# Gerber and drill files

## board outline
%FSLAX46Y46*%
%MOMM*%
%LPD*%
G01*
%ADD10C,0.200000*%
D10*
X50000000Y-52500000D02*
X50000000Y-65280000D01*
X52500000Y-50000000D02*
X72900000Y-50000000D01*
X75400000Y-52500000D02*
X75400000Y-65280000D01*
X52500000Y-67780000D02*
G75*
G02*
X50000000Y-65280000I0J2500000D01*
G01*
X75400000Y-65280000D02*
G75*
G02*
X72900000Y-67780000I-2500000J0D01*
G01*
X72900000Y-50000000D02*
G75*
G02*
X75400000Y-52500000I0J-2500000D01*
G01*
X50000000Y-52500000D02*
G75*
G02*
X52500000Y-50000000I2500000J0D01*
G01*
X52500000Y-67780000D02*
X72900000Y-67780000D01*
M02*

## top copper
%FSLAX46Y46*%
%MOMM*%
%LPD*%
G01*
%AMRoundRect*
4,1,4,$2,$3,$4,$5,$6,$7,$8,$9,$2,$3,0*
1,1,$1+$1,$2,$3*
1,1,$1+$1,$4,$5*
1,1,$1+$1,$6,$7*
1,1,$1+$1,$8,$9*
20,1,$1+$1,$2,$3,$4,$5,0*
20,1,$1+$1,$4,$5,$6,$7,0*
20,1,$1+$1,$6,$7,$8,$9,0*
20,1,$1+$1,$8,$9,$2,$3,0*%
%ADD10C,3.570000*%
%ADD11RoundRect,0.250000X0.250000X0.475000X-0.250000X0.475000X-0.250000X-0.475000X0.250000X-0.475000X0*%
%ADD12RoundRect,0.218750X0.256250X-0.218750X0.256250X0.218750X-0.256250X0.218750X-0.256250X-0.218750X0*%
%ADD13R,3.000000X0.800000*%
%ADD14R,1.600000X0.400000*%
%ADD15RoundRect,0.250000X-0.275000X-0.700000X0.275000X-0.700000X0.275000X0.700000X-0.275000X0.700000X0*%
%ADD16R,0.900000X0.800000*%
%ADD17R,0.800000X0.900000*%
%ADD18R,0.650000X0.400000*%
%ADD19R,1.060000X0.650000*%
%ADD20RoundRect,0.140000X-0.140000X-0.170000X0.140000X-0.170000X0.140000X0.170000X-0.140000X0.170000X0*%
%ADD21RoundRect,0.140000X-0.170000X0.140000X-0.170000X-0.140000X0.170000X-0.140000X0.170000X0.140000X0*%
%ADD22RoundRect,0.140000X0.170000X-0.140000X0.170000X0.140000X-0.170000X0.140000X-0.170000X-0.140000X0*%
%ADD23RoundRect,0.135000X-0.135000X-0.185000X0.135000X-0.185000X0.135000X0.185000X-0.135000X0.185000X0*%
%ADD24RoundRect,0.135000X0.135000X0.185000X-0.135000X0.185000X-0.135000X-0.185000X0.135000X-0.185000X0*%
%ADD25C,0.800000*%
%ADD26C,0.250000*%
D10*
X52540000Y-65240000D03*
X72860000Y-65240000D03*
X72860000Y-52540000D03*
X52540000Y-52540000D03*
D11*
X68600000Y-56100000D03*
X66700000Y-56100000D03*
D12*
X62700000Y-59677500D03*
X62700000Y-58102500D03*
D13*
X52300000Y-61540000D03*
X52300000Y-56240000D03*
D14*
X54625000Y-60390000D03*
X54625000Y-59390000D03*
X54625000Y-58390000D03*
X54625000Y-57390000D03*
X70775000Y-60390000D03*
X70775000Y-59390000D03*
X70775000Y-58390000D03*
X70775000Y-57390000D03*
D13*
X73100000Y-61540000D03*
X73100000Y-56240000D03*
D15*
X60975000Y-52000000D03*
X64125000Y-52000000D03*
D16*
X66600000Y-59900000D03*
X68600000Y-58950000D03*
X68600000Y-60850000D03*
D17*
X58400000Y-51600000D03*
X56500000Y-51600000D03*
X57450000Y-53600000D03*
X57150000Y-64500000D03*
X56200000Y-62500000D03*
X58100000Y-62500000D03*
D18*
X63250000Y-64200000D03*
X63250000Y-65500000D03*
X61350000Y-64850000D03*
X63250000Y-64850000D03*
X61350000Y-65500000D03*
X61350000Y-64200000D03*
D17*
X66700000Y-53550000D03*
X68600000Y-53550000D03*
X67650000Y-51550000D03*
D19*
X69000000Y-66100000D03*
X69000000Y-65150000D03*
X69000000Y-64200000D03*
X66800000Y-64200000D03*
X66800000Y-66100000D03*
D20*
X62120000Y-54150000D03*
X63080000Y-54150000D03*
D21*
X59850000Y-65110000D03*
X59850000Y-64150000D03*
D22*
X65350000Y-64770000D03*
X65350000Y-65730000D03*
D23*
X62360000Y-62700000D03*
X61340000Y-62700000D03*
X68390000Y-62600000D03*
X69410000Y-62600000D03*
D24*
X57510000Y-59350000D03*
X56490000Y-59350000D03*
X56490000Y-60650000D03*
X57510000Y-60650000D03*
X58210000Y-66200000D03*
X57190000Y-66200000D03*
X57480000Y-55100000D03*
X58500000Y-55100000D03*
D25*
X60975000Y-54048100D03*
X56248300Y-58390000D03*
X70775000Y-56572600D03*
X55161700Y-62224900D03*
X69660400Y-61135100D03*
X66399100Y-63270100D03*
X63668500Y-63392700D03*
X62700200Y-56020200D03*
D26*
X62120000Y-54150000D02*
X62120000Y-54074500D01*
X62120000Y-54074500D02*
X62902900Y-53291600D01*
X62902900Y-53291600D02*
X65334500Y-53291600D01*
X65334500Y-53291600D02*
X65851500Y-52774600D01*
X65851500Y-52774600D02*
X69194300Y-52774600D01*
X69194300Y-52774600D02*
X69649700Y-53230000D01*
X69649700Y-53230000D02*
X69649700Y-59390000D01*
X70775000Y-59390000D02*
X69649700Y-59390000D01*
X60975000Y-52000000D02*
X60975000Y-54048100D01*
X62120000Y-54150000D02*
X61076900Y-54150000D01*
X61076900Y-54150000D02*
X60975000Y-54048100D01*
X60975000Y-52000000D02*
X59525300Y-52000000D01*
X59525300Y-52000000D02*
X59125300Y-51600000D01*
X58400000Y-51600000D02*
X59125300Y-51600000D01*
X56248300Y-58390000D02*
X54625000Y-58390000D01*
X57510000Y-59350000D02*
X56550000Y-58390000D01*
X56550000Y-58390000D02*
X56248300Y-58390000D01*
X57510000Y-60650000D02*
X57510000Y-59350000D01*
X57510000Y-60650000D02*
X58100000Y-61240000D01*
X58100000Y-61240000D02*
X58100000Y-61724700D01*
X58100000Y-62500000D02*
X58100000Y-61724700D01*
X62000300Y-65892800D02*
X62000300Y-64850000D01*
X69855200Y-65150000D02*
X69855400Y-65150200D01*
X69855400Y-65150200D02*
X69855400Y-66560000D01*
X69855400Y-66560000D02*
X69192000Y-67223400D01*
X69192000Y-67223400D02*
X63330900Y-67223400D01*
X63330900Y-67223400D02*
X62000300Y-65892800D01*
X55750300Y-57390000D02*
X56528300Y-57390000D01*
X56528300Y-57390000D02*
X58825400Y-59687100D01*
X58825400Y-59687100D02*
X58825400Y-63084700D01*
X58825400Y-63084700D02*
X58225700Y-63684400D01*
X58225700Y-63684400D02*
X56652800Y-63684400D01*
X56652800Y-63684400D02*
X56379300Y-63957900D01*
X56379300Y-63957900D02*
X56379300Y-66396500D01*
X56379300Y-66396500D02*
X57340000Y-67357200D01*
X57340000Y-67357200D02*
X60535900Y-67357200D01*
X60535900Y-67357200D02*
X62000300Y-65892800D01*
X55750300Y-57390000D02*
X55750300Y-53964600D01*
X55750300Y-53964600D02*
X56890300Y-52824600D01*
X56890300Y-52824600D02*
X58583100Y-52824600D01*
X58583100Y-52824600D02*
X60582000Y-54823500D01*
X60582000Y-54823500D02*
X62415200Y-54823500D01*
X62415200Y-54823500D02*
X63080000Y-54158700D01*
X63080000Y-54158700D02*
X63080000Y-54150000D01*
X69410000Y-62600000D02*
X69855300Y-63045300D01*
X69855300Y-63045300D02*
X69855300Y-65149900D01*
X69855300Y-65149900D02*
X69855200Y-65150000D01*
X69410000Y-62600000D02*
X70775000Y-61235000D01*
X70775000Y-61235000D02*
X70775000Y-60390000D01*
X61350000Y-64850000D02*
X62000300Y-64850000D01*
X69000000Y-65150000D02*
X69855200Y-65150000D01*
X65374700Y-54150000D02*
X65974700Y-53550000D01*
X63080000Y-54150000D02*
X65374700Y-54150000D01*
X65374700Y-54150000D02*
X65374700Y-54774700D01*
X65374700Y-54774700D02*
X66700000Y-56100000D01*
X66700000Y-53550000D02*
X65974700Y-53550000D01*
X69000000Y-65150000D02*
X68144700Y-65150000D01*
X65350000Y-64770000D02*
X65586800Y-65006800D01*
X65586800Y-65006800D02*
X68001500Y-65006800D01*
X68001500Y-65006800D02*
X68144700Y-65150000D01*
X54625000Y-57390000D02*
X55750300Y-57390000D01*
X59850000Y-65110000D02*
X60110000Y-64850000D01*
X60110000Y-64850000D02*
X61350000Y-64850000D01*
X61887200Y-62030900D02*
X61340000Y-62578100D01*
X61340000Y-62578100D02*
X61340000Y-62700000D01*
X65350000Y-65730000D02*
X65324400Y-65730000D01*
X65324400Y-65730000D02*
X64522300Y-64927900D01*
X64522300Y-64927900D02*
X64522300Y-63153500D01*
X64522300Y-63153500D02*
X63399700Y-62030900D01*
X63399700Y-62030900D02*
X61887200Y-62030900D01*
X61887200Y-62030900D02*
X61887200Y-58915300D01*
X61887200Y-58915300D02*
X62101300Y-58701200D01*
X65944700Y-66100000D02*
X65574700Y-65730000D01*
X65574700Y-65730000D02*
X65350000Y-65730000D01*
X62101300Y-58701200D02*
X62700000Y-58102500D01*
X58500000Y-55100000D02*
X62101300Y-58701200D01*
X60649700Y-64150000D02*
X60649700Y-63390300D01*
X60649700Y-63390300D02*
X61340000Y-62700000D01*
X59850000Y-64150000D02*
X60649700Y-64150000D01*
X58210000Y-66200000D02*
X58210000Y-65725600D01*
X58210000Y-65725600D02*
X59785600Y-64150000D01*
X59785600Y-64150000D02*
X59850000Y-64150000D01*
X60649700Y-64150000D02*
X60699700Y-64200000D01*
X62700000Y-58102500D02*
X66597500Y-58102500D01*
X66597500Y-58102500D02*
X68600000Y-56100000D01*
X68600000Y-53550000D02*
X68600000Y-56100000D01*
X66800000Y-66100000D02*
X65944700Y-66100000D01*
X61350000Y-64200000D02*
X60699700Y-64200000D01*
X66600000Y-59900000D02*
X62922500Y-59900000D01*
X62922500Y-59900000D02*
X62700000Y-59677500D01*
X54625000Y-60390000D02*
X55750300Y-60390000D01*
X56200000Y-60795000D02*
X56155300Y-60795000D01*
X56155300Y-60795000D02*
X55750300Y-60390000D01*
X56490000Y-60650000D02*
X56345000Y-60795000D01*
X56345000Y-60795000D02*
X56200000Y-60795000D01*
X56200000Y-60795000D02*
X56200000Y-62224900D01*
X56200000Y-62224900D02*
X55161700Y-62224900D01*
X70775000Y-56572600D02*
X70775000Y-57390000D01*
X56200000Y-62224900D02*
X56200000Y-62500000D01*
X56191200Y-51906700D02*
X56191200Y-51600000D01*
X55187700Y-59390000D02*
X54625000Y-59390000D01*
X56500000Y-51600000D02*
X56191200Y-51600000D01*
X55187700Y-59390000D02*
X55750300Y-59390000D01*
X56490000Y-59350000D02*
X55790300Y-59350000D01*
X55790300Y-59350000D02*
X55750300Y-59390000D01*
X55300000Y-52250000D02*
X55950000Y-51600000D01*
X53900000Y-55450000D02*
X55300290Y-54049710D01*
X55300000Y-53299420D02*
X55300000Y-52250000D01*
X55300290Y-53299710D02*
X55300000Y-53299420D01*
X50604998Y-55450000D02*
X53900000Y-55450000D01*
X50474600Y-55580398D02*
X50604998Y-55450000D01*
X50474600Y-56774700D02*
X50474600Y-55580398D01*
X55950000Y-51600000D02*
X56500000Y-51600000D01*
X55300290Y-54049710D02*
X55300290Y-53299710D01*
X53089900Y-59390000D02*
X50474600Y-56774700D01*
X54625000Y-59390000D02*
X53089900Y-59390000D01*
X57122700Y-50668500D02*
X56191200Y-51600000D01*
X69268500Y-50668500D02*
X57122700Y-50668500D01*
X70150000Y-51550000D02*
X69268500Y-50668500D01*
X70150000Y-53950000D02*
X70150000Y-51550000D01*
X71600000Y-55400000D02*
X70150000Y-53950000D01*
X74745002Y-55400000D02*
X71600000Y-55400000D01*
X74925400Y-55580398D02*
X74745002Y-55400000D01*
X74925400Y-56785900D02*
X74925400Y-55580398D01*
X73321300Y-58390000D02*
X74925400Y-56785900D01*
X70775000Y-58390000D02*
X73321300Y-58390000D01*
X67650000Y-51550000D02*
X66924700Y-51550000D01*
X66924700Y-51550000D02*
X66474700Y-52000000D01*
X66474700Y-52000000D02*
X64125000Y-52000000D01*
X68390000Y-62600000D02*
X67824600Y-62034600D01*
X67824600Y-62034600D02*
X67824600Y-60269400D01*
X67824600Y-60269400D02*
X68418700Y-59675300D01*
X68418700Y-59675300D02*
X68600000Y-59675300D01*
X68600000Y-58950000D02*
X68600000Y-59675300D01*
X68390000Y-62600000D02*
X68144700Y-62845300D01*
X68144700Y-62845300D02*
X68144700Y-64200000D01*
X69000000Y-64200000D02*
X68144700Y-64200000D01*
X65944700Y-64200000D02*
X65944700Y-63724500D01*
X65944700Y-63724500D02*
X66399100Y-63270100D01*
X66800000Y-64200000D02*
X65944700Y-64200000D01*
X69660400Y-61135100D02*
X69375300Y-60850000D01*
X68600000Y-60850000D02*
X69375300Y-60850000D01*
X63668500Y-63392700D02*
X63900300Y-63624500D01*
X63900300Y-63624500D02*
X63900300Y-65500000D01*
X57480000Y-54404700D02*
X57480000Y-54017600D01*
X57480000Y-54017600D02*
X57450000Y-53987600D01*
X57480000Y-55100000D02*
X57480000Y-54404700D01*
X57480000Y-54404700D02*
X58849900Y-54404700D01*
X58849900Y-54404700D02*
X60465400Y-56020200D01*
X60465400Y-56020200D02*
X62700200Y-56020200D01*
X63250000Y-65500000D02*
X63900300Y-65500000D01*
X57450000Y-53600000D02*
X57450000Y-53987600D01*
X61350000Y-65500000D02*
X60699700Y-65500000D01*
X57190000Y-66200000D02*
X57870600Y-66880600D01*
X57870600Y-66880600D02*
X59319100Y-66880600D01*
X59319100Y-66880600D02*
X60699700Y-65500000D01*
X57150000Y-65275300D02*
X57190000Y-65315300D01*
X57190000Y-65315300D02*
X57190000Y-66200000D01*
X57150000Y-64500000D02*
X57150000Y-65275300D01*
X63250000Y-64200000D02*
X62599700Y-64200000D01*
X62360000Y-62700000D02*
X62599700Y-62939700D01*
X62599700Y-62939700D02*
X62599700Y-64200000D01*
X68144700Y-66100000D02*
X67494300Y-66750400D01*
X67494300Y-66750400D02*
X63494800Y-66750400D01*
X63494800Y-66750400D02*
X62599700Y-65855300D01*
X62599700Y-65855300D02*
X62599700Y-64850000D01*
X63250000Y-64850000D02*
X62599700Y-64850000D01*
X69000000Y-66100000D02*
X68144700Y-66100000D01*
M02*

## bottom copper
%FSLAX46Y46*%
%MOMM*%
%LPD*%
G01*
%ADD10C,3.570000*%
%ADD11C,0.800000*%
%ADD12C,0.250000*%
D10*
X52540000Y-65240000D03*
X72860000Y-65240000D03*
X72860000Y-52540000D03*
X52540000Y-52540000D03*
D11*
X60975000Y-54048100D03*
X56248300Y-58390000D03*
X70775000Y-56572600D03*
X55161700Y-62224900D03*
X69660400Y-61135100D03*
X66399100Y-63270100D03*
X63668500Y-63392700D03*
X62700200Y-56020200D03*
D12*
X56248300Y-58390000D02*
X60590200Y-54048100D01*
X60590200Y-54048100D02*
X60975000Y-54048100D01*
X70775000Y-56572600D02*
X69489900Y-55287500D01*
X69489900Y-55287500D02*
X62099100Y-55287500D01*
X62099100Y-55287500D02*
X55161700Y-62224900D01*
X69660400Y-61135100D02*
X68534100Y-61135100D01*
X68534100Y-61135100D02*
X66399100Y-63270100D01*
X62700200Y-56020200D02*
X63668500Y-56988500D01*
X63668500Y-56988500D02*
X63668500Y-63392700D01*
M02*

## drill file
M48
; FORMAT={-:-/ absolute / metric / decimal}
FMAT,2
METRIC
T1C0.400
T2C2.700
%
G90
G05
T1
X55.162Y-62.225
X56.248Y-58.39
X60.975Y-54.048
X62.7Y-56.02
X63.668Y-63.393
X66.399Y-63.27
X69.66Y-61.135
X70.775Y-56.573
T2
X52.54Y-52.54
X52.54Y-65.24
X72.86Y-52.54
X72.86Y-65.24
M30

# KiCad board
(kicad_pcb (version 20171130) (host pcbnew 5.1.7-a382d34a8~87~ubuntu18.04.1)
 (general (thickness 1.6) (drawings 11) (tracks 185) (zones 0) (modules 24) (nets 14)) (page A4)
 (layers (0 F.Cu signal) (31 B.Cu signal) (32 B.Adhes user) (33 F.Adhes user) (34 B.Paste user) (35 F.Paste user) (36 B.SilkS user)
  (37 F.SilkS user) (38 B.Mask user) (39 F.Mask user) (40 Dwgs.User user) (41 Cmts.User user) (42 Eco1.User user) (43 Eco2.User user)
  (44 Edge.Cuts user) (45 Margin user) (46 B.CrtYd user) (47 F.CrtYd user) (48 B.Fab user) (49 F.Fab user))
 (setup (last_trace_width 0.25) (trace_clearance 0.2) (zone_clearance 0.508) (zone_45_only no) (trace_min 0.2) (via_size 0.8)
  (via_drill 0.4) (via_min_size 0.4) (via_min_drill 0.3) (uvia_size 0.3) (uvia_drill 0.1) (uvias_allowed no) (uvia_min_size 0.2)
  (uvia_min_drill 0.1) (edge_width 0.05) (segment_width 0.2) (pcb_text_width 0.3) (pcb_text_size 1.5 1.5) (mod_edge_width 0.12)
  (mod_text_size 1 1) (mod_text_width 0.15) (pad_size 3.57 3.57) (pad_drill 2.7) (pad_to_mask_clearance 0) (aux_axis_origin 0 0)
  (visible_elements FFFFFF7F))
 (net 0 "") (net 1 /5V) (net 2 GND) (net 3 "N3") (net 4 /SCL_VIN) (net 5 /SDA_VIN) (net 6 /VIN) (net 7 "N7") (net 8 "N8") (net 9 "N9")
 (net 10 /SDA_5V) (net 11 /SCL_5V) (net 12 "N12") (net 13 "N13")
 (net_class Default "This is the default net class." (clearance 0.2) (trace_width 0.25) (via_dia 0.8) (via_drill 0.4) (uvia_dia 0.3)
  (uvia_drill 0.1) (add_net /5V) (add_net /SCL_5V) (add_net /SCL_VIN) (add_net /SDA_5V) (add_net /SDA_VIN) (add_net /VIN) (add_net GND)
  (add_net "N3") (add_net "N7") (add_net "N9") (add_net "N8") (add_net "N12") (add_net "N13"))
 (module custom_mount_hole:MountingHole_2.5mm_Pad (layer F.Cu) (at 52.54 65.24)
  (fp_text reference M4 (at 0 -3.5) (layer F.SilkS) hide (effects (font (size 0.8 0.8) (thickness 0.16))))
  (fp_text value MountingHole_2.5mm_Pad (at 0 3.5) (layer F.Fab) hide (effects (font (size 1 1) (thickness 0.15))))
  (pad ~ thru_hole circle (at 0 0) (size 3.57 3.57) (drill 2.7) (layers *.Cu *.Mask)))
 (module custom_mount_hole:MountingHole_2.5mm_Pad (layer F.Cu) (at 72.86 65.24)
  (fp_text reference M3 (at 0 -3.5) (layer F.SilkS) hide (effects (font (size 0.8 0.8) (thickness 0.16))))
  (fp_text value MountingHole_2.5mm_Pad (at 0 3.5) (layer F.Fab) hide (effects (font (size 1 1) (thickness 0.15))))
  (pad ~ thru_hole circle (at 0 0) (size 3.57 3.57) (drill 2.7) (layers *.Cu *.Mask)))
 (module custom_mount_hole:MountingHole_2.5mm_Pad (layer F.Cu) (at 72.86 52.54)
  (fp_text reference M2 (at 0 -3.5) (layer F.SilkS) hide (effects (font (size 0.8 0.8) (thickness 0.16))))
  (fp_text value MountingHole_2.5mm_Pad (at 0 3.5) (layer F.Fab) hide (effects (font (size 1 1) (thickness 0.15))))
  (pad ~ thru_hole circle (at 0 0) (size 3.57 3.57) (drill 2.7) (layers *.Cu *.Mask)))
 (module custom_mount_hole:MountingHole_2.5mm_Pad (layer F.Cu) (at 52.54 52.54)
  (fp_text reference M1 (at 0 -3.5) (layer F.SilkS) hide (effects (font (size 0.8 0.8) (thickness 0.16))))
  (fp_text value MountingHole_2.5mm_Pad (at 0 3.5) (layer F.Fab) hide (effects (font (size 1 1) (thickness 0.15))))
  (pad ~ thru_hole circle (at 0 0) (size 3.57 3.57) (drill 2.7) (layers *.Cu *.Mask)))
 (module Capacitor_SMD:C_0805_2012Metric (layer F.Cu) (at 67.65 56.1 180)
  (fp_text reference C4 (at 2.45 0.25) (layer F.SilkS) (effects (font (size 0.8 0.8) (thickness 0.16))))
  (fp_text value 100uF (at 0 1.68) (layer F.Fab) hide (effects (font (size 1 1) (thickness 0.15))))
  (pad 1 smd roundrect (at -0.95 0 180) (size 1 1.45) (layers F.Cu F.Paste F.Mask) (roundrect_rratio 0.25) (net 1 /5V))
  (pad 2 smd roundrect (at 0.95 0 180) (size 1 1.45) (layers F.Cu F.Paste F.Mask) (roundrect_rratio 0.25) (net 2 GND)))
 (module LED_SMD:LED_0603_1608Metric (layer F.Cu) (at 62.7 58.89 90)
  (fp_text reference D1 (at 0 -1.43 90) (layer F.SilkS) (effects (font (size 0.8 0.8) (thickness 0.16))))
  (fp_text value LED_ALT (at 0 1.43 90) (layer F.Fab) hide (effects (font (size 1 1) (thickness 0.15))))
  (pad 1 smd roundrect (at -0.7875 0 90) (size 0.875 0.95) (layers F.Cu F.Paste F.Mask) (roundrect_rratio 0.25) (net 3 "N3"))
  (pad 2 smd roundrect (at 0.7875 0 90) (size 0.875 0.95) (layers F.Cu F.Paste F.Mask) (roundrect_rratio 0.25) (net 1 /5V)))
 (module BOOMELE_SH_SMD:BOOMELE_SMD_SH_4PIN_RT (layer F.Cu) (at 52.3 58.89 270)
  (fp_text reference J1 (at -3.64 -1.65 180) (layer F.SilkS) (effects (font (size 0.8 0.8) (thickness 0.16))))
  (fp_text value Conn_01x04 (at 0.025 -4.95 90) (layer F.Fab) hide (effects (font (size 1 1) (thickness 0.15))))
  (pad "" smd rect (at 2.65 0 270) (size 0.8 3) (layers F.Cu F.Paste F.Mask))
  (pad "" smd rect (at -2.65 0 270) (size 0.8 3) (layers F.Cu F.Paste F.Mask))
  (pad 4 smd rect (at 1.5 -2.325 270) (size 0.4 1.6) (layers F.Cu F.Paste F.Mask) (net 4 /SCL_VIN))
  (pad 3 smd rect (at 0.5 -2.325 270) (size 0.4 1.6) (layers F.Cu F.Paste F.Mask) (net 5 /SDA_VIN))
  (pad 2 smd rect (at -0.5 -2.325 270) (size 0.4 1.6) (layers F.Cu F.Paste F.Mask) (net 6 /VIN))
  (pad 1 smd rect (at -1.5 -2.325 270) (size 0.4 1.6) (layers F.Cu F.Paste F.Mask) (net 2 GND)))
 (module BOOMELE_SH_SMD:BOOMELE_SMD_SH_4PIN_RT (layer F.Cu) (at 73.1 58.89 90)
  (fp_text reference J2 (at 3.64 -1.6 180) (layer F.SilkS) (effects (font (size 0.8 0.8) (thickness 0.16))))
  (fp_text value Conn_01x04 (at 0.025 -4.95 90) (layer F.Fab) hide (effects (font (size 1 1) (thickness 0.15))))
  (pad 1 smd rect (at -1.5 -2.325 90) (size 0.4 1.6) (layers F.Cu F.Paste F.Mask) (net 2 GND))
  (pad 2 smd rect (at -0.5 -2.325 90) (size 0.4 1.6) (layers F.Cu F.Paste F.Mask) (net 6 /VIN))
  (pad 3 smd rect (at 0.5 -2.325 90) (size 0.4 1.6) (layers F.Cu F.Paste F.Mask) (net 5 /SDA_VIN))
  (pad 4 smd rect (at 1.5 -2.325 90) (size 0.4 1.6) (layers F.Cu F.Paste F.Mask) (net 4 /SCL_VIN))
  (pad "" smd rect (at -2.65 0 90) (size 0.8 3) (layers F.Cu F.Paste F.Mask))
  (pad "" smd rect (at 2.65 0 90) (size 0.8 3) (layers F.Cu F.Paste F.Mask)))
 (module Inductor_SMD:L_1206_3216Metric (layer F.Cu) (at 62.55 52)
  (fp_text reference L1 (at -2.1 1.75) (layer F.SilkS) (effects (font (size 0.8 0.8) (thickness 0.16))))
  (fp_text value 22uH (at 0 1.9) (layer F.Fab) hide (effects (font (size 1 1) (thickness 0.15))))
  (pad 1 smd roundrect (at -1.575 0) (size 1.05 1.9) (layers F.Cu F.Paste F.Mask) (roundrect_rratio 0.238095) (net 6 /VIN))
  (pad 2 smd roundrect (at 1.575 0) (size 1.05 1.9) (layers F.Cu F.Paste F.Mask) (roundrect_rratio 0.238095) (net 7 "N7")))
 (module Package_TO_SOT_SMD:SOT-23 (layer F.Cu) (at 67.6 59.9 180)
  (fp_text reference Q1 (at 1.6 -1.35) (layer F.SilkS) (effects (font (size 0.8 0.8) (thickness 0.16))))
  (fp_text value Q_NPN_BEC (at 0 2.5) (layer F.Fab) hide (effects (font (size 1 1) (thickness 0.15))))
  (pad 3 smd rect (at 1 0 180) (size 0.9 0.8) (layers F.Cu F.Paste F.Mask) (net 3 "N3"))
  (pad 2 smd rect (at -1 0.95 180) (size 0.9 0.8) (layers F.Cu F.Paste F.Mask) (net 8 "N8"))
  (pad 1 smd rect (at -1 -0.95 180) (size 0.9 0.8) (layers F.Cu F.Paste F.Mask) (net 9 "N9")))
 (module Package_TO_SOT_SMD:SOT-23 (layer F.Cu) (at 57.45 52.6 270)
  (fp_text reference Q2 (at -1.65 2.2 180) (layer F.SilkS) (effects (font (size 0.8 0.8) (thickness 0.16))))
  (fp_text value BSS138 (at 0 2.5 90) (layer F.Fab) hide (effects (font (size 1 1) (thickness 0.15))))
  (pad 1 smd rect (at -1 -0.95 270) (size 0.9 0.8) (layers F.Cu F.Paste F.Mask) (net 6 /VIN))
  (pad 2 smd rect (at -1 0.95 270) (size 0.9 0.8) (layers F.Cu F.Paste F.Mask) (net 5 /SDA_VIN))
  (pad 3 smd rect (at 1 0 270) (size 0.9 0.8) (layers F.Cu F.Paste F.Mask) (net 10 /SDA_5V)))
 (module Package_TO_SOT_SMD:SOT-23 (layer F.Cu) (at 57.15 63.5 270)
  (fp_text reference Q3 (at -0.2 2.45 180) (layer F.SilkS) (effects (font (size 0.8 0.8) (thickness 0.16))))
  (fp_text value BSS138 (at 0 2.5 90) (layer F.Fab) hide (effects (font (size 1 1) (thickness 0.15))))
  (pad 3 smd rect (at 1 0 270) (size 0.9 0.8) (layers F.Cu F.Paste F.Mask) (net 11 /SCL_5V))
  (pad 2 smd rect (at -1 0.95 270) (size 0.9 0.8) (layers F.Cu F.Paste F.Mask) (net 4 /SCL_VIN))
  (pad 1 smd rect (at -1 -0.95 270) (size 0.9 0.8) (layers F.Cu F.Paste F.Mask) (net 6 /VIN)))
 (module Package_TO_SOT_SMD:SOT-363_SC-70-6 (layer F.Cu) (at 62.3 64.85)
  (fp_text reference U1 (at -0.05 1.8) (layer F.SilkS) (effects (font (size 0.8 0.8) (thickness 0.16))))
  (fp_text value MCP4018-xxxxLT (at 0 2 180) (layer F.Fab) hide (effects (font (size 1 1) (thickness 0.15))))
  (pad 6 smd rect (at 0.95 -0.65) (size 0.65 0.4) (layers F.Cu F.Paste F.Mask) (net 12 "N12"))
  (pad 4 smd rect (at 0.95 0.65) (size 0.65 0.4) (layers F.Cu F.Paste F.Mask) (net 10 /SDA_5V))
  (pad 2 smd rect (at -0.95 0) (size 0.65 0.4) (layers F.Cu F.Paste F.Mask) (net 2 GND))
  (pad 5 smd rect (at 0.95 0) (size 0.65 0.4) (layers F.Cu F.Paste F.Mask) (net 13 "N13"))
  (pad 3 smd rect (at -0.95 0.65) (size 0.65 0.4) (layers F.Cu F.Paste F.Mask) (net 11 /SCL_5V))
  (pad 1 smd rect (at -0.95 -0.65) (size 0.65 0.4) (layers F.Cu F.Paste F.Mask) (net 1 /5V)))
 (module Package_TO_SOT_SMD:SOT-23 (layer F.Cu) (at 67.65 52.55 90)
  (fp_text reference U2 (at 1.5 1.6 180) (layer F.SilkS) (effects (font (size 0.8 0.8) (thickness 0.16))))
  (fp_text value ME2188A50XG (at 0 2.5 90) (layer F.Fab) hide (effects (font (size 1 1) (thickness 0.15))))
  (pad 1 smd rect (at -1 -0.95 90) (size 0.9 0.8) (layers F.Cu F.Paste F.Mask) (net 2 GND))
  (pad 2 smd rect (at -1 0.95 90) (size 0.9 0.8) (layers F.Cu F.Paste F.Mask) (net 1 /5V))
  (pad 3 smd rect (at 1 0 90) (size 0.9 0.8) (layers F.Cu F.Paste F.Mask) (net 7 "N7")))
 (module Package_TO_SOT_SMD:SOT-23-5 (layer F.Cu) (at 67.9 65.15 180)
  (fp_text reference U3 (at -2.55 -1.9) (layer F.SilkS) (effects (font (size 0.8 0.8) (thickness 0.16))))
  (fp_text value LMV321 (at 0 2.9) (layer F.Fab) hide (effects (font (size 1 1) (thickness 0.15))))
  (pad 1 smd rect (at -1.1 -0.95 180) (size 1.06 0.65) (layers F.Cu F.Paste F.Mask) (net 13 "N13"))
  (pad 2 smd rect (at -1.1 0 180) (size 1.06 0.65) (layers F.Cu F.Paste F.Mask) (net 2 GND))
  (pad 3 smd rect (at -1.1 0.95 180) (size 1.06 0.65) (layers F.Cu F.Paste F.Mask) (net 8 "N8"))
  (pad 4 smd rect (at 1.1 0.95 180) (size 1.06 0.65) (layers F.Cu F.Paste F.Mask) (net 9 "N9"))
  (pad 5 smd rect (at 1.1 -0.95 180) (size 1.06 0.65) (layers F.Cu F.Paste F.Mask) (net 1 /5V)))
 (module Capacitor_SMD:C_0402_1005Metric (layer F.Cu) (at 62.6 54.15)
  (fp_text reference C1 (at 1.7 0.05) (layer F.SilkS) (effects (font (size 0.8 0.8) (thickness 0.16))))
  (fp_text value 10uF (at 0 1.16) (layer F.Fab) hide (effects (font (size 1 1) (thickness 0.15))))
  (pad 1 smd roundrect (at -0.48 0) (size 0.56 0.62) (layers F.Cu F.Paste F.Mask) (roundrect_rratio 0.25) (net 6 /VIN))
  (pad 2 smd roundrect (at 0.48 0) (size 0.56 0.62) (layers F.Cu F.Paste F.Mask) (roundrect_rratio 0.25) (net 2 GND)))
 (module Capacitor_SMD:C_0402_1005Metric (layer F.Cu) (at 59.85 64.63 270)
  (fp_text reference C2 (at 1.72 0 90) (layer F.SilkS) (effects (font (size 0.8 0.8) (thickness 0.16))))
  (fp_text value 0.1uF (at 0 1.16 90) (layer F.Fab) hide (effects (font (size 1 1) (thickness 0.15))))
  (pad 2 smd roundrect (at 0.48 0 270) (size 0.56 0.62) (layers F.Cu F.Paste F.Mask) (roundrect_rratio 0.25) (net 2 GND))
  (pad 1 smd roundrect (at -0.48 0 270) (size 0.56 0.62) (layers F.Cu F.Paste F.Mask) (roundrect_rratio 0.25) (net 1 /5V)))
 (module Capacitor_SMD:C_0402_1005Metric (layer F.Cu) (at 65.35 65.25 90)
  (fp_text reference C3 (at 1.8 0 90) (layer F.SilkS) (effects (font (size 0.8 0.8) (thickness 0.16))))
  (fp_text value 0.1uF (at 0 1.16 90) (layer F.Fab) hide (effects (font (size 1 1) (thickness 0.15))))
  (pad 2 smd roundrect (at 0.48 0 90) (size 0.56 0.62) (layers F.Cu F.Paste F.Mask) (roundrect_rratio 0.25) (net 2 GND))
  (pad 1 smd roundrect (at -0.48 0 90) (size 0.56 0.62) (layers F.Cu F.Paste F.Mask) (roundrect_rratio 0.25) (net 1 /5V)))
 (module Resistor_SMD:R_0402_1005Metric (layer F.Cu) (at 61.85 62.7)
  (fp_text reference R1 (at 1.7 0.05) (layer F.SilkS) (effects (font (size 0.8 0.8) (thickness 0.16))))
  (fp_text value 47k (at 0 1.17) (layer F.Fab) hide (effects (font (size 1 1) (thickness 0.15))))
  (pad 2 smd roundrect (at 0.51 0) (size 0.54 0.64) (layers F.Cu F.Paste F.Mask) (roundrect_rratio 0.25) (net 12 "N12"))
  (pad 1 smd roundrect (at -0.51 0) (size 0.54 0.64) (layers F.Cu F.Paste F.Mask) (roundrect_rratio 0.25) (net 1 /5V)))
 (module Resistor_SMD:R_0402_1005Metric (layer F.Cu) (at 68.9 62.6)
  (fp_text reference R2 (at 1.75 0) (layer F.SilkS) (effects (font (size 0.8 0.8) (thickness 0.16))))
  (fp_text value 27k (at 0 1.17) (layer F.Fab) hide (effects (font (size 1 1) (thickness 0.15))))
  (pad 1 smd roundrect (at -0.51 0) (size 0.54 0.64) (layers F.Cu F.Paste F.Mask) (roundrect_rratio 0.25) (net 8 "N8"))
  (pad 2 smd roundrect (at 0.51 0) (size 0.54 0.64) (layers F.Cu F.Paste F.Mask) (roundrect_rratio 0.25) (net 2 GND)))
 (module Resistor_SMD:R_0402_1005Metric (layer F.Cu) (at 57 59.35 180)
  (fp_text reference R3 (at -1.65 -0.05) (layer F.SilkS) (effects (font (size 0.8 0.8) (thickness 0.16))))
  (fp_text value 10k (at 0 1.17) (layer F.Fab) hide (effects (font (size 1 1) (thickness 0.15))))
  (pad 1 smd roundrect (at -0.51 0 180) (size 0.54 0.64) (layers F.Cu F.Paste F.Mask) (roundrect_rratio 0.25) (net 6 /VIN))
  (pad 2 smd roundrect (at 0.51 0 180) (size 0.54 0.64) (layers F.Cu F.Paste F.Mask) (roundrect_rratio 0.25) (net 5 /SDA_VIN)))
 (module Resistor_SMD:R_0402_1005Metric (layer F.Cu) (at 57 60.65 180)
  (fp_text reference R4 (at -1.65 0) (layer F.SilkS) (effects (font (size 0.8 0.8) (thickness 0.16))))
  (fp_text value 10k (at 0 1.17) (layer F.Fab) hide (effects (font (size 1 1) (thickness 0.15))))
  (pad 2 smd roundrect (at 0.51 0 180) (size 0.54 0.64) (layers F.Cu F.Paste F.Mask) (roundrect_rratio 0.25) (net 4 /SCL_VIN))
  (pad 1 smd roundrect (at -0.51 0 180) (size 0.54 0.64) (layers F.Cu F.Paste F.Mask) (roundrect_rratio 0.25) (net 6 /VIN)))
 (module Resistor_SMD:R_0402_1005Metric (layer F.Cu) (at 57.7 66.2 180)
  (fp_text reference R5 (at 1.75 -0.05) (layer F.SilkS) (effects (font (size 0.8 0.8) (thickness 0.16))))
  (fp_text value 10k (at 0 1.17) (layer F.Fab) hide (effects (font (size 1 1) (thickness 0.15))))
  (pad 1 smd roundrect (at -0.51 0 180) (size 0.54 0.64) (layers F.Cu F.Paste F.Mask) (roundrect_rratio 0.25) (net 1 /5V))
  (pad 2 smd roundrect (at 0.51 0 180) (size 0.54 0.64) (layers F.Cu F.Paste F.Mask) (roundrect_rratio 0.25) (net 11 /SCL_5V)))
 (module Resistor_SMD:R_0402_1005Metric (layer F.Cu) (at 57.99 55.1 180)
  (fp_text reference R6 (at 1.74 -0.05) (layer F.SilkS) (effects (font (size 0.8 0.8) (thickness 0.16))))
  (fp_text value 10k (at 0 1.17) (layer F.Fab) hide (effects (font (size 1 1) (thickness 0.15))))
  (pad 2 smd roundrect (at 0.51 0 180) (size 0.54 0.64) (layers F.Cu F.Paste F.Mask) (roundrect_rratio 0.25) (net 10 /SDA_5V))
  (pad 1 smd roundrect (at -0.51 0 180) (size 0.54 0.64) (layers F.Cu F.Paste F.Mask) (roundrect_rratio 0.25) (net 1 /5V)))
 (gr_line (start 50 52.5) (end 50 65.28) (layer Edge.Cuts) (width 0.2))
 (gr_line (start 52.5 50) (end 72.9 50) (layer Edge.Cuts) (width 0.2))
 (gr_line (start 75.4 52.5) (end 75.4 65.28) (layer Edge.Cuts) (width 0.2))
 (gr_arc (start 52.5 65.28) (end 50 65.28) (angle -90) (layer Edge.Cuts) (width 0.2))
 (gr_arc (start 72.9 65.28) (end 72.9 67.78) (angle -90) (layer Edge.Cuts) (width 0.2))
 (gr_arc (start 72.9 52.5) (end 75.4 52.5) (angle -90) (layer Edge.Cuts) (width 0.2))
 (gr_arc (start 52.5 52.5) (end 52.5 50) (angle -90) (layer Edge.Cuts) (width 0.2))
 (gr_line (start 52.5 67.78) (end 72.9 67.78) (layer Edge.Cuts) (width 0.2))
 (segment (start 62.12 54.15) (end 62.12 54.0745) (width 0.25) (layer F.Cu) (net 6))
 (segment (start 62.12 54.0745) (end 62.9029 53.2916) (width 0.25) (layer F.Cu) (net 6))
 (segment (start 62.9029 53.2916) (end 65.3345 53.2916) (width 0.25) (layer F.Cu) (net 6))
 (segment (start 65.3345 53.2916) (end 65.8515 52.7746) (width 0.25) (layer F.Cu) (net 6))
 (segment (start 65.8515 52.7746) (end 69.1943 52.7746) (width 0.25) (layer F.Cu) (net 6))
 (segment (start 69.1943 52.7746) (end 69.6497 53.23) (width 0.25) (layer F.Cu) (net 6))
 (segment (start 69.6497 53.23) (end 69.6497 59.39) (width 0.25) (layer F.Cu) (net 6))
 (segment (start 56.2483 58.39) (end 60.5902 54.0481) (width 0.25) (layer B.Cu) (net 6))
 (segment (start 60.5902 54.0481) (end 60.975 54.0481) (width 0.25) (layer B.Cu) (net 6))
 (segment (start 70.775 59.39) (end 69.6497 59.39) (width 0.25) (layer F.Cu) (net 6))
 (segment (start 60.975 52) (end 60.975 54.0481) (width 0.25) (layer F.Cu) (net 6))
 (segment (start 62.12 54.15) (end 61.0769 54.15) (width 0.25) (layer F.Cu) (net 6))
 (segment (start 61.0769 54.15) (end 60.975 54.0481) (width 0.25) (layer F.Cu) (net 6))
 (segment (start 60.975 52) (end 59.5253 52) (width 0.25) (layer F.Cu) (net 6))
 (segment (start 59.5253 52) (end 59.1253 51.6) (width 0.25) (layer F.Cu) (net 6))
 (segment (start 58.4 51.6) (end 59.1253 51.6) (width 0.25) (layer F.Cu) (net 6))
 (segment (start 56.2483 58.39) (end 54.625 58.39) (width 0.25) (layer F.Cu) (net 6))
 (segment (start 57.51 59.35) (end 56.55 58.39) (width 0.25) (layer F.Cu) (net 6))
 (segment (start 56.55 58.39) (end 56.2483 58.39) (width 0.25) (layer F.Cu) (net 6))
 (segment (start 57.51 60.65) (end 57.51 59.35) (width 0.25) (layer F.Cu) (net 6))
 (segment (start 57.51 60.65) (end 58.1 61.24) (width 0.25) (layer F.Cu) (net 6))
 (segment (start 58.1 61.24) (end 58.1 61.7247) (width 0.25) (layer F.Cu) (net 6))
 (segment (start 58.1 62.5) (end 58.1 61.7247) (width 0.25) (layer F.Cu) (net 6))
 (via (at 60.975 54.0481) (size 0.8) (layers F.Cu B.Cu) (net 6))
 (via (at 56.2483 58.39) (size 0.8) (layers F.Cu B.Cu) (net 6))
 (segment (start 62.0003 65.8928) (end 62.0003 64.85) (width 0.25) (layer F.Cu) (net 2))
 (segment (start 69.8552 65.15) (end 69.8554 65.1502) (width 0.25) (layer F.Cu) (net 2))
 (segment (start 69.8554 65.1502) (end 69.8554 66.56) (width 0.25) (layer F.Cu) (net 2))
 (segment (start 69.8554 66.56) (end 69.192 67.2234) (width 0.25) (layer F.Cu) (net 2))
 (segment (start 69.192 67.2234) (end 63.3309 67.2234) (width 0.25) (layer F.Cu) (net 2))
 (segment (start 63.3309 67.2234) (end 62.0003 65.8928) (width 0.25) (layer F.Cu) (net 2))
 (segment (start 55.7503 57.39) (end 56.5283 57.39) (width 0.25) (layer F.Cu) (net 2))
 (segment (start 56.5283 57.39) (end 58.8254 59.6871) (width 0.25) (layer F.Cu) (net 2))
 (segment (start 58.8254 59.6871) (end 58.8254 63.0847) (width 0.25) (layer F.Cu) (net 2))
 (segment (start 58.8254 63.0847) (end 58.2257 63.6844) (width 0.25) (layer F.Cu) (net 2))
 (segment (start 58.2257 63.6844) (end 56.6528 63.6844) (width 0.25) (layer F.Cu) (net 2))
 (segment (start 56.6528 63.6844) (end 56.3793 63.9579) (width 0.25) (layer F.Cu) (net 2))
 (segment (start 56.3793 63.9579) (end 56.3793 66.3965) (width 0.25) (layer F.Cu) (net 2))
 (segment (start 56.3793 66.3965) (end 57.34 67.3572) (width 0.25) (layer F.Cu) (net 2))
 (segment (start 57.34 67.3572) (end 60.5359 67.3572) (width 0.25) (layer F.Cu) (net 2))
 (segment (start 60.5359 67.3572) (end 62.0003 65.8928) (width 0.25) (layer F.Cu) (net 2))
 (segment (start 55.7503 57.39) (end 55.7503 53.9646) (width 0.25) (layer F.Cu) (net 2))
 (segment (start 55.7503 53.9646) (end 56.8903 52.8246) (width 0.25) (layer F.Cu) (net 2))
 (segment (start 56.8903 52.8246) (end 58.5831 52.8246) (width 0.25) (layer F.Cu) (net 2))
 (segment (start 58.5831 52.8246) (end 60.582 54.8235) (width 0.25) (layer F.Cu) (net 2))
 (segment (start 60.582 54.8235) (end 62.4152 54.8235) (width 0.25) (layer F.Cu) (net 2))
 (segment (start 62.4152 54.8235) (end 63.08 54.1587) (width 0.25) (layer F.Cu) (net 2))
 (segment (start 63.08 54.1587) (end 63.08 54.15) (width 0.25) (layer F.Cu) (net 2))
 (segment (start 69.41 62.6) (end 69.8553 63.0453) (width 0.25) (layer F.Cu) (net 2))
 (segment (start 69.8553 63.0453) (end 69.8553 65.1499) (width 0.25) (layer F.Cu) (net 2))
 (segment (start 69.8553 65.1499) (end 69.8552 65.15) (width 0.25) (layer F.Cu) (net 2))
 (segment (start 69.41 62.6) (end 70.775 61.235) (width 0.25) (layer F.Cu) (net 2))
 (segment (start 70.775 61.235) (end 70.775 60.39) (width 0.25) (layer F.Cu) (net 2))
 (segment (start 61.35 64.85) (end 62.0003 64.85) (width 0.25) (layer F.Cu) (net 2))
 (segment (start 69 65.15) (end 69.8552 65.15) (width 0.25) (layer F.Cu) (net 2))
 (segment (start 65.3747 54.15) (end 65.9747 53.55) (width 0.25) (layer F.Cu) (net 2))
 (segment (start 63.08 54.15) (end 65.3747 54.15) (width 0.25) (layer F.Cu) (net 2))
 (segment (start 65.3747 54.15) (end 65.3747 54.7747) (width 0.25) (layer F.Cu) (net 2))
 (segment (start 65.3747 54.7747) (end 66.7 56.1) (width 0.25) (layer F.Cu) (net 2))
 (segment (start 66.7 53.55) (end 65.9747 53.55) (width 0.25) (layer F.Cu) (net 2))
 (segment (start 69 65.15) (end 68.1447 65.15) (width 0.25) (layer F.Cu) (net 2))
 (segment (start 65.35 64.77) (end 65.5868 65.0068) (width 0.25) (layer F.Cu) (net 2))
 (segment (start 65.5868 65.0068) (end 68.0015 65.0068) (width 0.25) (layer F.Cu) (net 2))
 (segment (start 68.0015 65.0068) (end 68.1447 65.15) (width 0.25) (layer F.Cu) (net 2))
 (segment (start 54.625 57.39) (end 55.7503 57.39) (width 0.25) (layer F.Cu) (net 2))
 (segment (start 59.85 65.11) (end 60.11 64.85) (width 0.25) (layer F.Cu) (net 2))
 (segment (start 60.11 64.85) (end 61.35 64.85) (width 0.25) (layer F.Cu) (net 2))
 (segment (start 61.8872 62.0309) (end 61.34 62.5781) (width 0.25) (layer F.Cu) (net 1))
 (segment (start 61.34 62.5781) (end 61.34 62.7) (width 0.25) (layer F.Cu) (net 1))
 (segment (start 65.35 65.73) (end 65.3244 65.73) (width 0.25) (layer F.Cu) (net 1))
 (segment (start 65.3244 65.73) (end 64.5223 64.9279) (width 0.25) (layer F.Cu) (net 1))
 (segment (start 64.5223 64.9279) (end 64.5223 63.1535) (width 0.25) (layer F.Cu) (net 1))
 (segment (start 64.5223 63.1535) (end 63.3997 62.0309) (width 0.25) (layer F.Cu) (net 1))
 (segment (start 63.3997 62.0309) (end 61.8872 62.0309) (width 0.25) (layer F.Cu) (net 1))
 (segment (start 61.8872 62.0309) (end 61.8872 58.9153) (width 0.25) (layer F.Cu) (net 1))
 (segment (start 61.8872 58.9153) (end 62.1013 58.7012) (width 0.25) (layer F.Cu) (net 1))
 (segment (start 65.9447 66.1) (end 65.5747 65.73) (width 0.25) (layer F.Cu) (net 1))
 (segment (start 65.5747 65.73) (end 65.35 65.73) (width 0.25) (layer F.Cu) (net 1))
 (segment (start 62.1013 58.7012) (end 62.7 58.1025) (width 0.25) (layer F.Cu) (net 1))
 (segment (start 58.5 55.1) (end 62.1013 58.7012) (width 0.25) (layer F.Cu) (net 1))
 (segment (start 60.6497 64.15) (end 60.6497 63.3903) (width 0.25) (layer F.Cu) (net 1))
 (segment (start 60.6497 63.3903) (end 61.34 62.7) (width 0.25) (layer F.Cu) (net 1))
 (segment (start 59.85 64.15) (end 60.6497 64.15) (width 0.25) (layer F.Cu) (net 1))
 (segment (start 58.21 66.2) (end 58.21 65.7256) (width 0.25) (layer F.Cu) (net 1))
 (segment (start 58.21 65.7256) (end 59.7856 64.15) (width 0.25) (layer F.Cu) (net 1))
 (segment (start 59.7856 64.15) (end 59.85 64.15) (width 0.25) (layer F.Cu) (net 1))
 (segment (start 60.6497 64.15) (end 60.6997 64.2) (width 0.25) (layer F.Cu) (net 1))
 (segment (start 62.7 58.1025) (end 66.5975 58.1025) (width 0.25) (layer F.Cu) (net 1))
 (segment (start 66.5975 58.1025) (end 68.6 56.1) (width 0.25) (layer F.Cu) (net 1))
 (segment (start 68.6 53.55) (end 68.6 56.1) (width 0.25) (layer F.Cu) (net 1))
 (segment (start 66.8 66.1) (end 65.9447 66.1) (width 0.25) (layer F.Cu) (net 1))
 (segment (start 61.35 64.2) (end 60.6997 64.2) (width 0.25) (layer F.Cu) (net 1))
 (segment (start 66.6 59.9) (end 62.9225 59.9) (width 0.25) (layer F.Cu) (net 3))
 (segment (start 62.9225 59.9) (end 62.7 59.6775) (width 0.25) (layer F.Cu) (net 3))
 (segment (start 54.625 60.39) (end 55.7503 60.39) (width 0.25) (layer F.Cu) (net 4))
 (segment (start 56.2 60.795) (end 56.1553 60.795) (width 0.25) (layer F.Cu) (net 4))
 (segment (start 56.1553 60.795) (end 55.7503 60.39) (width 0.25) (layer F.Cu) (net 4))
 (segment (start 56.49 60.65) (end 56.345 60.795) (width 0.25) (layer F.Cu) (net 4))
 (segment (start 56.345 60.795) (end 56.2 60.795) (width 0.25) (layer F.Cu) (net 4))
 (segment (start 56.2 60.795) (end 56.2 62.2249) (width 0.25) (layer F.Cu) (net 4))
 (segment (start 56.2 62.2249) (end 55.1617 62.2249) (width 0.25) (layer F.Cu) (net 4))
 (segment (start 70.775 56.5726) (end 69.4899 55.2875) (width 0.25) (layer B.Cu) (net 4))
 (segment (start 69.4899 55.2875) (end 62.0991 55.2875) (width 0.25) (layer B.Cu) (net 4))
 (segment (start 62.0991 55.2875) (end 55.1617 62.2249) (width 0.25) (layer B.Cu) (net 4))
 (segment (start 70.775 56.5726) (end 70.775 57.39) (width 0.25) (layer F.Cu) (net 4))
 (segment (start 56.2 62.2249) (end 56.2 62.5) (width 0.25) (layer F.Cu) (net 4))
 (via (at 70.775 56.5726) (size 0.8) (layers F.Cu B.Cu) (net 4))
 (via (at 55.1617 62.2249) (size 0.8) (layers F.Cu B.Cu) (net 4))
 (segment (start 56.1912 51.9067) (end 56.1912 51.6) (width 0.25) (layer F.Cu) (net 5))
 (segment (start 55.1877 59.39) (end 54.625 59.39) (width 0.25) (layer F.Cu) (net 5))
 (segment (start 56.5 51.6) (end 56.1912 51.6) (width 0.25) (layer F.Cu) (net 5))
 (segment (start 55.1877 59.39) (end 55.7503 59.39) (width 0.25) (layer F.Cu) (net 5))
 (segment (start 56.49 59.35) (end 55.7903 59.35) (width 0.25) (layer F.Cu) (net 5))
 (segment (start 55.7903 59.35) (end 55.7503 59.39) (width 0.25) (layer F.Cu) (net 5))
 (segment (start 55.3 52.25) (end 55.95 51.6) (width 0.25) (layer F.Cu) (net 5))
 (segment (start 53.9 55.45) (end 55.30029 54.04971) (width 0.25) (layer F.Cu) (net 5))
 (segment (start 55.3 53.29942) (end 55.3 52.25) (width 0.25) (layer F.Cu) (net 5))
 (segment (start 55.30029 53.29971) (end 55.3 53.29942) (width 0.25) (layer F.Cu) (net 5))
 (segment (start 50.604998 55.45) (end 53.9 55.45) (width 0.25) (layer F.Cu) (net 5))
 (segment (start 50.4746 55.580398) (end 50.604998 55.45) (width 0.25) (layer F.Cu) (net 5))
 (segment (start 50.4746 56.7747) (end 50.4746 55.580398) (width 0.25) (layer F.Cu) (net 5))
 (segment (start 55.95 51.6) (end 56.5 51.6) (width 0.25) (layer F.Cu) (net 5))
 (segment (start 55.30029 54.04971) (end 55.30029 53.29971) (width 0.25) (layer F.Cu) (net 5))
 (segment (start 53.0899 59.39) (end 50.4746 56.7747) (width 0.25) (layer F.Cu) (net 5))
 (segment (start 54.625 59.39) (end 53.0899 59.39) (width 0.25) (layer F.Cu) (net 5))
 (segment (start 57.1227 50.6685) (end 56.1912 51.6) (width 0.25) (layer F.Cu) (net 5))
 (segment (start 69.2685 50.6685) (end 57.1227 50.6685) (width 0.25) (layer F.Cu) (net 5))
 (segment (start 70.15 51.55) (end 69.2685 50.6685) (width 0.25) (layer F.Cu) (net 5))
 (segment (start 70.15 53.95) (end 70.15 51.55) (width 0.25) (layer F.Cu) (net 5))
 (segment (start 71.6 55.4) (end 70.15 53.95) (width 0.25) (layer F.Cu) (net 5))
 (segment (start 74.745002 55.4) (end 71.6 55.4) (width 0.25) (layer F.Cu) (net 5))
 (segment (start 74.9254 55.580398) (end 74.745002 55.4) (width 0.25) (layer F.Cu) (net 5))
 (segment (start 74.9254 56.7859) (end 74.9254 55.580398) (width 0.25) (layer F.Cu) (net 5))
 (segment (start 73.3213 58.39) (end 74.9254 56.7859) (width 0.25) (layer F.Cu) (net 5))
 (segment (start 70.775 58.39) (end 73.3213 58.39) (width 0.25) (layer F.Cu) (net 5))
 (segment (start 67.65 51.55) (end 66.9247 51.55) (width 0.25) (layer F.Cu) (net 7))
 (segment (start 66.9247 51.55) (end 66.4747 52) (width 0.25) (layer F.Cu) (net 7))
 (segment (start 66.4747 52) (end 64.125 52) (width 0.25) (layer F.Cu) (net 7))
 (segment (start 68.39 62.6) (end 67.8246 62.0346) (width 0.25) (layer F.Cu) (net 8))
 (segment (start 67.8246 62.0346) (end 67.8246 60.2694) (width 0.25) (layer F.Cu) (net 8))
 (segment (start 67.8246 60.2694) (end 68.4187 59.6753) (width 0.25) (layer F.Cu) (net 8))
 (segment (start 68.4187 59.6753) (end 68.6 59.6753) (width 0.25) (layer F.Cu) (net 8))
 (segment (start 68.6 58.95) (end 68.6 59.6753) (width 0.25) (layer F.Cu) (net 8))
 (segment (start 68.39 62.6) (end 68.1447 62.8453) (width 0.25) (layer F.Cu) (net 8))
 (segment (start 68.1447 62.8453) (end 68.1447 64.2) (width 0.25) (layer F.Cu) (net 8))
 (segment (start 69 64.2) (end 68.1447 64.2) (width 0.25) (layer F.Cu) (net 8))
 (segment (start 65.9447 64.2) (end 65.9447 63.7245) (width 0.25) (layer F.Cu) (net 9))
 (segment (start 65.9447 63.7245) (end 66.3991 63.2701) (width 0.25) (layer F.Cu) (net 9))
 (segment (start 69.6604 61.1351) (end 68.5341 61.1351) (width 0.25) (layer B.Cu) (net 9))
 (segment (start 68.5341 61.1351) (end 66.3991 63.2701) (width 0.25) (layer B.Cu) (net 9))
 (segment (start 66.8 64.2) (end 65.9447 64.2) (width 0.25) (layer F.Cu) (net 9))
 (segment (start 69.6604 61.1351) (end 69.3753 60.85) (width 0.25) (layer F.Cu) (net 9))
 (segment (start 68.6 60.85) (end 69.3753 60.85) (width 0.25) (layer F.Cu) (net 9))
 (via (at 69.6604 61.1351) (size 0.8) (layers F.Cu B.Cu) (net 9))
 (via (at 66.3991 63.2701) (size 0.8) (layers F.Cu B.Cu) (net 9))
 (segment (start 63.6685 63.3927) (end 63.9003 63.6245) (width 0.25) (layer F.Cu) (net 10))
 (segment (start 63.9003 63.6245) (end 63.9003 65.5) (width 0.25) (layer F.Cu) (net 10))
 (segment (start 62.7002 56.0202) (end 63.6685 56.9885) (width 0.25) (layer B.Cu) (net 10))
 (segment (start 63.6685 56.9885) (end 63.6685 63.3927) (width 0.25) (layer B.Cu) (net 10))
 (segment (start 57.48 54.4047) (end 57.48 54.0176) (width 0.25) (layer F.Cu) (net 10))
 (segment (start 57.48 54.0176) (end 57.45 53.9876) (width 0.25) (layer F.Cu) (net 10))
 (segment (start 57.48 55.1) (end 57.48 54.4047) (width 0.25) (layer F.Cu) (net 10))
 (segment (start 57.48 54.4047) (end 58.8499 54.4047) (width 0.25) (layer F.Cu) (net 10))
 (segment (start 58.8499 54.4047) (end 60.4654 56.0202) (width 0.25) (layer F.Cu) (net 10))
 (segment (start 60.4654 56.0202) (end 62.7002 56.0202) (width 0.25) (layer F.Cu) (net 10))
 (segment (start 63.25 65.5) (end 63.9003 65.5) (width 0.25) (layer F.Cu) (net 10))
 (segment (start 57.45 53.6) (end 57.45 53.9876) (width 0.25) (layer F.Cu) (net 10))
 (via (at 63.6685 63.3927) (size 0.8) (layers F.Cu B.Cu) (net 10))
 (via (at 62.7002 56.0202) (size 0.8) (layers F.Cu B.Cu) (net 10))
 (segment (start 61.35 65.5) (end 60.6997 65.5) (width 0.25) (layer F.Cu) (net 11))
 (segment (start 57.19 66.2) (end 57.8706 66.8806) (width 0.25) (layer F.Cu) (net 11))
 (segment (start 57.8706 66.8806) (end 59.3191 66.8806) (width 0.25) (layer F.Cu) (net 11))
 (segment (start 59.3191 66.8806) (end 60.6997 65.5) (width 0.25) (layer F.Cu) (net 11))
 (segment (start 57.15 65.2753) (end 57.19 65.3153) (width 0.25) (layer F.Cu) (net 11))
 (segment (start 57.19 65.3153) (end 57.19 66.2) (width 0.25) (layer F.Cu) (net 11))
 (segment (start 57.15 64.5) (end 57.15 65.2753) (width 0.25) (layer F.Cu) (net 11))
 (segment (start 63.25 64.2) (end 62.5997 64.2) (width 0.25) (layer F.Cu) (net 12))
 (segment (start 62.36 62.7) (end 62.5997 62.9397) (width 0.25) (layer F.Cu) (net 12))
 (segment (start 62.5997 62.9397) (end 62.5997 64.2) (width 0.25) (layer F.Cu) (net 12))
 (segment (start 68.1447 66.1) (end 67.4943 66.7504) (width 0.25) (layer F.Cu) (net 13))
 (segment (start 67.4943 66.7504) (end 63.4948 66.7504) (width 0.25) (layer F.Cu) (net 13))
 (segment (start 63.4948 66.7504) (end 62.5997 65.8553) (width 0.25) (layer F.Cu) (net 13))
 (segment (start 62.5997 65.8553) (end 62.5997 64.85) (width 0.25) (layer F.Cu) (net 13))
 (segment (start 63.25 64.85) (end 62.5997 64.85) (width 0.25) (layer F.Cu) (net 13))
 (segment (start 69 66.1) (end 68.1447 66.1) (width 0.25) (layer F.Cu) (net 13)))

